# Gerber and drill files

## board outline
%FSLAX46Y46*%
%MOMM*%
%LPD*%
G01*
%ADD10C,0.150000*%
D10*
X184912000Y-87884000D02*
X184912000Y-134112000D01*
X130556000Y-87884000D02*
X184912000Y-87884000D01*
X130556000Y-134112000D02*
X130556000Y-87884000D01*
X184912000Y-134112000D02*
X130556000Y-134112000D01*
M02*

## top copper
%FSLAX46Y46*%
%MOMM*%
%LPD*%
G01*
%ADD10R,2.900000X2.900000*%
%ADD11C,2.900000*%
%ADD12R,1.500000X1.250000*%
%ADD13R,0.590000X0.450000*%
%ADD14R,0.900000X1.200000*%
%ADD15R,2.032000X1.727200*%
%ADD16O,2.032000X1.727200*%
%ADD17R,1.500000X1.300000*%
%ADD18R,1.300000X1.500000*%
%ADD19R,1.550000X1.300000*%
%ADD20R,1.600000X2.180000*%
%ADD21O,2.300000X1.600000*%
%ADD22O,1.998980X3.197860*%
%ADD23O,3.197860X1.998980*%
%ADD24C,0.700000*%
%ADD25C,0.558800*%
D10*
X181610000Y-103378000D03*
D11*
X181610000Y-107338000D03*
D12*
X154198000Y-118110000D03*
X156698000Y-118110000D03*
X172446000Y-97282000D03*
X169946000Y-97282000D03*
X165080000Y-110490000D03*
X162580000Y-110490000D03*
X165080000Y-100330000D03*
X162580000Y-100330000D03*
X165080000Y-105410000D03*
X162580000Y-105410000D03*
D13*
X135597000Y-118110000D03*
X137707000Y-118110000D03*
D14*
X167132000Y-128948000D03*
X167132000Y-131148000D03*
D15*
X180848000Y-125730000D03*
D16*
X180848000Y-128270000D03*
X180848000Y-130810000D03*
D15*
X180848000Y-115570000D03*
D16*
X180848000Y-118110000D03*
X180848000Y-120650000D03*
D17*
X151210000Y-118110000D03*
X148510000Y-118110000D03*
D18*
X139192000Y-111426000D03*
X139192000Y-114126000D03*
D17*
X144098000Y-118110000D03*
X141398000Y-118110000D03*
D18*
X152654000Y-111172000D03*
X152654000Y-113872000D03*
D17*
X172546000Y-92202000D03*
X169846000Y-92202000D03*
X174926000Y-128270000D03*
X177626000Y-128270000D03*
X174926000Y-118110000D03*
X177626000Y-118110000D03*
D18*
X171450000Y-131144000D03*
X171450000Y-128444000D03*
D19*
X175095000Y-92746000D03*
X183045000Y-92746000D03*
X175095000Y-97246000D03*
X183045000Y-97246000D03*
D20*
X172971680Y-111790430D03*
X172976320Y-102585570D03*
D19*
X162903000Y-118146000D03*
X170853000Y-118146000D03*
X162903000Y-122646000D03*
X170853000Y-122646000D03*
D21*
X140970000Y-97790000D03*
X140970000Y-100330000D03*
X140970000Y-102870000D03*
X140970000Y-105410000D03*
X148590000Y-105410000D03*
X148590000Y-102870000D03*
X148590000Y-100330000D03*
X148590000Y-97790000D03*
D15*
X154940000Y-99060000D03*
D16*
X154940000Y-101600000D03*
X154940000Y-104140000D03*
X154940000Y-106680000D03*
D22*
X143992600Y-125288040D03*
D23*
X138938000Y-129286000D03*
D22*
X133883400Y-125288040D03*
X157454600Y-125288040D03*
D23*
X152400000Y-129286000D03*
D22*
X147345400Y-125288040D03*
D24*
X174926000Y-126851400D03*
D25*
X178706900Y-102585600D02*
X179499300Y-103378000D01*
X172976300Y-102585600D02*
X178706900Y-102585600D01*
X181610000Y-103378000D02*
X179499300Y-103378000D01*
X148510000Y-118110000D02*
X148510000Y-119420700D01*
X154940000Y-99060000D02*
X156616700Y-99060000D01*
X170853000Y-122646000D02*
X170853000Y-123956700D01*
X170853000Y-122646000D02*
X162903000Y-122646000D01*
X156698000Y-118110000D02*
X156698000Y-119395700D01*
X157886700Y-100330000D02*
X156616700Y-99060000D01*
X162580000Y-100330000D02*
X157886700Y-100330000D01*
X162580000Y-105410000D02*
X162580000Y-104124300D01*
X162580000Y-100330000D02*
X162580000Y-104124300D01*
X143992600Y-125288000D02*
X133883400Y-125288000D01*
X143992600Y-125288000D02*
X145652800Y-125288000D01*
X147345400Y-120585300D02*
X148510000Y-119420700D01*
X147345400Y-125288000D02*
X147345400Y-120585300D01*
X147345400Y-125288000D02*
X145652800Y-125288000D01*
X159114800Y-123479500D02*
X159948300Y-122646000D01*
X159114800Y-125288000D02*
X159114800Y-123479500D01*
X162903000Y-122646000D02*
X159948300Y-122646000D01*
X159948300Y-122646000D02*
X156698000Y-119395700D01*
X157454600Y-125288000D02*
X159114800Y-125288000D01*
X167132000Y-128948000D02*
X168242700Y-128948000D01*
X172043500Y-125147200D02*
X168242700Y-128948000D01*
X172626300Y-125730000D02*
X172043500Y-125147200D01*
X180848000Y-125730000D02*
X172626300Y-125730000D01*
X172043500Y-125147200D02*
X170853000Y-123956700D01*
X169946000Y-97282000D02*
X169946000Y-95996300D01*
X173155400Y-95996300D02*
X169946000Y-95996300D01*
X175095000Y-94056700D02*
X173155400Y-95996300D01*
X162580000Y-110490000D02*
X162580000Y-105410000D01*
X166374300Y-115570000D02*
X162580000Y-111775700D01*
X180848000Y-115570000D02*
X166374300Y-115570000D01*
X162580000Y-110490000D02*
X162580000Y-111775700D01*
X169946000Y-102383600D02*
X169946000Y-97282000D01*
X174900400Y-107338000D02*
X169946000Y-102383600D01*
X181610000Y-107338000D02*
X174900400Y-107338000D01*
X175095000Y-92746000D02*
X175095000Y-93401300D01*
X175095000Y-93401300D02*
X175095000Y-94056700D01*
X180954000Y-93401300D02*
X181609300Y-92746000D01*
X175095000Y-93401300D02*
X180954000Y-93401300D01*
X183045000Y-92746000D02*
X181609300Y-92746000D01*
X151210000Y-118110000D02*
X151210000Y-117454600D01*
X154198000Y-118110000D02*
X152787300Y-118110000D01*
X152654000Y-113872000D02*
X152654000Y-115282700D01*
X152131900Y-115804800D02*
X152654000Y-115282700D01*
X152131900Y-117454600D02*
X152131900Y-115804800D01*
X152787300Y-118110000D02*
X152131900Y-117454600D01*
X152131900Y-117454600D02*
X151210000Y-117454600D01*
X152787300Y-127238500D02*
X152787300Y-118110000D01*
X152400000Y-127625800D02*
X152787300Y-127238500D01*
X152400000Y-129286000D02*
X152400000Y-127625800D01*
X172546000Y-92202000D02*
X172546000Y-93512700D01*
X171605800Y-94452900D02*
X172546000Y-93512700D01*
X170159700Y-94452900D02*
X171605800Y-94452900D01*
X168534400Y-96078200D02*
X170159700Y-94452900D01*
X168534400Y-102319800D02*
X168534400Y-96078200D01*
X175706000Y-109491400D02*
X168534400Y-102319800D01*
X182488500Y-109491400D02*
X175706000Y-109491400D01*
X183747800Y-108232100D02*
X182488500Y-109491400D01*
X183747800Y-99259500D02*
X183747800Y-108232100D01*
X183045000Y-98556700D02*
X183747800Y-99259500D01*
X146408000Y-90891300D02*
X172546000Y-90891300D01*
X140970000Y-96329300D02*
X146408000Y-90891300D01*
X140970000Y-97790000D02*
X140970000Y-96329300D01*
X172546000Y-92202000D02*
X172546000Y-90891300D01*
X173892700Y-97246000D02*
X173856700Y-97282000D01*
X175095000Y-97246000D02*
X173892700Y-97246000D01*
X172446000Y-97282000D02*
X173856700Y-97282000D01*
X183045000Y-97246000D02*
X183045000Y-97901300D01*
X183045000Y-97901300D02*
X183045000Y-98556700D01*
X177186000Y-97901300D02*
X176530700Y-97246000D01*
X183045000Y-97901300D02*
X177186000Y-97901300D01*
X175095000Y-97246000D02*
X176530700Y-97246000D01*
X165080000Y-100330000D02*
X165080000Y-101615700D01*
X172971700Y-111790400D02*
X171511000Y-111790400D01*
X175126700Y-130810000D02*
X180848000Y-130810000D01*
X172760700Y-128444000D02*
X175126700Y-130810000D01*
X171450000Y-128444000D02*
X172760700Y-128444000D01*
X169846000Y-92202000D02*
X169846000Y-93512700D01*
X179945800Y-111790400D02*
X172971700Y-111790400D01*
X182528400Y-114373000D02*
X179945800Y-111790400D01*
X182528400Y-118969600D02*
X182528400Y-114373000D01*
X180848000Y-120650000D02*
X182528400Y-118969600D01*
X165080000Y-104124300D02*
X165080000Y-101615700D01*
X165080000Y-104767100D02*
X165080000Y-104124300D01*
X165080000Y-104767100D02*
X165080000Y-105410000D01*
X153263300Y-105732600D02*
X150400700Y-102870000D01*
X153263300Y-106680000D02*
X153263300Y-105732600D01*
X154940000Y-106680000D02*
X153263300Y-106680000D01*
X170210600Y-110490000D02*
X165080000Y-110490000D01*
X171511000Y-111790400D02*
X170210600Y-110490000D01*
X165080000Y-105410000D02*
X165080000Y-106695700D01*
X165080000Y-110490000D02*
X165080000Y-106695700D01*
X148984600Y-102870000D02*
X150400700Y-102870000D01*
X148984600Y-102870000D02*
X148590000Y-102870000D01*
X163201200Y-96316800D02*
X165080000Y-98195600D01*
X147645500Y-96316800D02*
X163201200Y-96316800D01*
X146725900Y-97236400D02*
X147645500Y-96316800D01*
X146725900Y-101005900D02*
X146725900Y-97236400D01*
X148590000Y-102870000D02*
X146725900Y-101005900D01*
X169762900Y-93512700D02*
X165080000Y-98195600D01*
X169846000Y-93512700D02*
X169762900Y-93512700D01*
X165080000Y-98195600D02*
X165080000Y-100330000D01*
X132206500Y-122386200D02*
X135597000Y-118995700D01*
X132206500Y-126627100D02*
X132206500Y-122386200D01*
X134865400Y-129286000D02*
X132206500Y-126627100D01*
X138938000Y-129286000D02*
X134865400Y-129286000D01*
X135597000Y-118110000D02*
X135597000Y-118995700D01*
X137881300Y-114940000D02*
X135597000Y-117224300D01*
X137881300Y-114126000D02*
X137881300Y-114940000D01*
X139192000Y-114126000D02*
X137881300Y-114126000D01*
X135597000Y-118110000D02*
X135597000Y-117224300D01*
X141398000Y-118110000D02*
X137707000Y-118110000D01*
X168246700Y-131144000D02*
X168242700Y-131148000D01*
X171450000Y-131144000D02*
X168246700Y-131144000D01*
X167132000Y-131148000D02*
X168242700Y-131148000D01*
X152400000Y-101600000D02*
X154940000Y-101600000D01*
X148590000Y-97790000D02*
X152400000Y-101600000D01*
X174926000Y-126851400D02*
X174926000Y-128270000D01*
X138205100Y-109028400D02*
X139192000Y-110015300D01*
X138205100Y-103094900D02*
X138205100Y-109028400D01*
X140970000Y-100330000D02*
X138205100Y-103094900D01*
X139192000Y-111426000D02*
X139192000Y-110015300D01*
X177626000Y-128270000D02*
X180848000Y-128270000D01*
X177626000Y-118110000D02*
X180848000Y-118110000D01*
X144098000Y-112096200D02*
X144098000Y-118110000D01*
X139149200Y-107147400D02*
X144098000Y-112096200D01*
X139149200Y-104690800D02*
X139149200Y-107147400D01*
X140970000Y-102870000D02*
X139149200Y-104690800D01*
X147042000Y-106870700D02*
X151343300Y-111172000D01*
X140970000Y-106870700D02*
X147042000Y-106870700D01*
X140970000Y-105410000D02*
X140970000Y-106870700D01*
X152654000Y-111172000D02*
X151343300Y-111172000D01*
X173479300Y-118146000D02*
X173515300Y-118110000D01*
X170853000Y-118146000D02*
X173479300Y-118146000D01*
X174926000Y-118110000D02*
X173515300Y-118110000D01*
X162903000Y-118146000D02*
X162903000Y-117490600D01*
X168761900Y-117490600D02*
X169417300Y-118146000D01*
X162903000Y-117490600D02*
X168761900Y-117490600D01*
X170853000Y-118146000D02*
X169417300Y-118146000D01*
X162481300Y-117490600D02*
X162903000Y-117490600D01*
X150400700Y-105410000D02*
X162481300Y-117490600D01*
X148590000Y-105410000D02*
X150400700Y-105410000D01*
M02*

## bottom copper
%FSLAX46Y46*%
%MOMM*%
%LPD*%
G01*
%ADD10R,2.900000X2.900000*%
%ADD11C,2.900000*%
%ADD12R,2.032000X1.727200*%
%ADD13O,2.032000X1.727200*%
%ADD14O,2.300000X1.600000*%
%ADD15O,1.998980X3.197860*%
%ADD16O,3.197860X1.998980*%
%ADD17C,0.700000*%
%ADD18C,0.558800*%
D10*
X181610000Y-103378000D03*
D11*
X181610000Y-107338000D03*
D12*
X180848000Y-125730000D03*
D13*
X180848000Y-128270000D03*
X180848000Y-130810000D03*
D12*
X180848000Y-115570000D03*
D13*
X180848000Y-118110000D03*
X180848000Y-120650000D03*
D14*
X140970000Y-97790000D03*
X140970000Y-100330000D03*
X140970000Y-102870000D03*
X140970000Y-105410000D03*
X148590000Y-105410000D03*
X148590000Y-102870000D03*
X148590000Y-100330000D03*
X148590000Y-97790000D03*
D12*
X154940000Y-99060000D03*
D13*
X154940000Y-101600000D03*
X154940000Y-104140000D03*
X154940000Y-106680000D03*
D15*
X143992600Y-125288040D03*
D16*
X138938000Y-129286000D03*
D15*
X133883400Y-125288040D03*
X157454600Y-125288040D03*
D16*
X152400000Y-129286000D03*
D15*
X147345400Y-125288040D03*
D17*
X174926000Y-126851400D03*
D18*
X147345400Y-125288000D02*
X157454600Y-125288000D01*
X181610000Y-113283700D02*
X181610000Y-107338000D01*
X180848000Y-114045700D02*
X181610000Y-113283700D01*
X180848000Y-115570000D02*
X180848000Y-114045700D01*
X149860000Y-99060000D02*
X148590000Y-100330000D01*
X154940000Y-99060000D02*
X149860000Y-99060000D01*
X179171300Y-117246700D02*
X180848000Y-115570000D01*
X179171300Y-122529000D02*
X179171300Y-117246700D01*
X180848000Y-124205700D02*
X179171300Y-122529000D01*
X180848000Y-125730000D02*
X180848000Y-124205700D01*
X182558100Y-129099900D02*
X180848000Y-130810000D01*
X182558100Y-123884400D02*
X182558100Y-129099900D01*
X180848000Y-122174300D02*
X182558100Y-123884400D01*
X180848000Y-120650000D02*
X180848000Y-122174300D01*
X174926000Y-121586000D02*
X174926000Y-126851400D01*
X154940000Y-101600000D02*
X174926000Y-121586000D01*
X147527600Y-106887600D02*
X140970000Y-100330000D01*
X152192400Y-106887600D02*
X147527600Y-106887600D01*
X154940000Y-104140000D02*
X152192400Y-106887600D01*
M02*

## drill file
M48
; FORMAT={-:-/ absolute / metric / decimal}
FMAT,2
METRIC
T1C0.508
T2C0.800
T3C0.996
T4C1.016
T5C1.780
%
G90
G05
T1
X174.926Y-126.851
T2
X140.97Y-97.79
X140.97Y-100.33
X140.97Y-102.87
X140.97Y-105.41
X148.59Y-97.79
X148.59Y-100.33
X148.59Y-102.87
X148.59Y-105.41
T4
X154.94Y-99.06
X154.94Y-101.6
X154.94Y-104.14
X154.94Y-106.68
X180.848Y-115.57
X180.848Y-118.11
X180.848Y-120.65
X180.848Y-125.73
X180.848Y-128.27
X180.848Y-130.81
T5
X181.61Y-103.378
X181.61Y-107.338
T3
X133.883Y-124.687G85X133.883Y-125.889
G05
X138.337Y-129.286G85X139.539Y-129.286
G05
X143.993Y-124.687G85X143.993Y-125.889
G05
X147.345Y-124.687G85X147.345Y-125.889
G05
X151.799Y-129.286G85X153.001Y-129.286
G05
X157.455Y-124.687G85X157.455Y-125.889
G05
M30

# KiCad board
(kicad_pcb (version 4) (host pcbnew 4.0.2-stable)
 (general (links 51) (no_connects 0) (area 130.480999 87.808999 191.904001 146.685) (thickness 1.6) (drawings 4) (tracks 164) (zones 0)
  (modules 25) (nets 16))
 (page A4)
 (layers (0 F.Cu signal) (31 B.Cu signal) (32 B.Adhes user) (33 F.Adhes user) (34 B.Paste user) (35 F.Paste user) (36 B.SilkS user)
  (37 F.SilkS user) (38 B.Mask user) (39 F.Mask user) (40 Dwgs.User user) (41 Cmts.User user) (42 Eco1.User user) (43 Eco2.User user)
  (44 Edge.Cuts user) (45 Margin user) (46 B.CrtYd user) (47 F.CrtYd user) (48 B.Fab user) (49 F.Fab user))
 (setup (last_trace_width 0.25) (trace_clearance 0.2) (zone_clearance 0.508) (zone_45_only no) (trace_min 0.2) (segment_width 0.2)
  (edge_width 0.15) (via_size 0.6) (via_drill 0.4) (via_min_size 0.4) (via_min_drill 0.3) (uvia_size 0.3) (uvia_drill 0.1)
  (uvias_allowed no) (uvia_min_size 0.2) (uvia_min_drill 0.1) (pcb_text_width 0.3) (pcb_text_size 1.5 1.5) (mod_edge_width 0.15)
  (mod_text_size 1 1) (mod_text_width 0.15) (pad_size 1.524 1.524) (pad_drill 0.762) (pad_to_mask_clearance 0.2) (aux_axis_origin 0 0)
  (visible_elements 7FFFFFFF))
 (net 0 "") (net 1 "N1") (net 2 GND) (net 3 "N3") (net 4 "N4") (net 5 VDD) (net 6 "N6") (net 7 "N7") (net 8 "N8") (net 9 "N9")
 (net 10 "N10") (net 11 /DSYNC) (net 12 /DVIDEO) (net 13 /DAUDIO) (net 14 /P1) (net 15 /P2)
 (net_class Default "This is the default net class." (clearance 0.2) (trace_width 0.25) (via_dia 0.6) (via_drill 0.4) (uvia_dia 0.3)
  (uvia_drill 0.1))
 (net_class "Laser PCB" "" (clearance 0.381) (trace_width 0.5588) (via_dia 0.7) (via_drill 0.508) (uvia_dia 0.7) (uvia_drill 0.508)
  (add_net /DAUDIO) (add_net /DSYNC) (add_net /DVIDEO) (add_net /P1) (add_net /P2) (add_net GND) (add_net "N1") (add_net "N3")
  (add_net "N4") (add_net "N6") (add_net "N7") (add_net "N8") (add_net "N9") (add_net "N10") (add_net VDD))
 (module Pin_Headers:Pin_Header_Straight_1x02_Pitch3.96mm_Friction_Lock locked (layer F.Cu) (at 181.61 103.378 270)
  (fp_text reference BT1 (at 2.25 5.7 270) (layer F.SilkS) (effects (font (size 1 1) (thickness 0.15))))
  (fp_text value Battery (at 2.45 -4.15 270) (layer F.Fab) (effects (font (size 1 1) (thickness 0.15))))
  (pad 1 thru_hole rect (at 0 0 270) (size 2.9 2.9) (drill 1.78) (layers *.Cu *.Mask F.SilkS) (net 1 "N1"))
  (pad 2 thru_hole circle (at 3.96 0 270) (size 2.9 2.9) (drill 1.78) (layers *.Cu *.Mask F.SilkS) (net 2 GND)))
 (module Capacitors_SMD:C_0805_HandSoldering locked (layer F.Cu) (at 155.448 118.11)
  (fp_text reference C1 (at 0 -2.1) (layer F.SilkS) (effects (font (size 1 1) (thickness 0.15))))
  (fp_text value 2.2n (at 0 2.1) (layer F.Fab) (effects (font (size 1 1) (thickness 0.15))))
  (pad 1 smd rect (at -1.25 0) (size 1.5 1.25) (layers F.Cu F.Paste F.Mask) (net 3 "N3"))
  (pad 2 smd rect (at 1.25 0) (size 1.5 1.25) (layers F.Cu F.Paste F.Mask) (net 2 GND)))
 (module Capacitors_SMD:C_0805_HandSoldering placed (layer F.Cu) (at 171.196 97.282 180)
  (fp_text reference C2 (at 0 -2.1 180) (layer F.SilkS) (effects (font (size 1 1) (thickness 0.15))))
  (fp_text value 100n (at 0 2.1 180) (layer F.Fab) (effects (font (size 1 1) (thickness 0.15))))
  (pad 1 smd rect (at -1.25 0 180) (size 1.5 1.25) (layers F.Cu F.Paste F.Mask) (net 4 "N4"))
  (pad 2 smd rect (at 1.25 0 180) (size 1.5 1.25) (layers F.Cu F.Paste F.Mask) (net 2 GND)))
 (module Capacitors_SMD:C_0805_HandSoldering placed (layer F.Cu) (at 163.83 110.49 180)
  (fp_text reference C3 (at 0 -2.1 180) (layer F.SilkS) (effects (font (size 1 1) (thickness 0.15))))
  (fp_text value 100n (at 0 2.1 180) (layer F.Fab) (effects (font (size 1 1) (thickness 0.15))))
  (pad 1 smd rect (at -1.25 0 180) (size 1.5 1.25) (layers F.Cu F.Paste F.Mask) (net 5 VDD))
  (pad 2 smd rect (at 1.25 0 180) (size 1.5 1.25) (layers F.Cu F.Paste F.Mask) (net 2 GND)))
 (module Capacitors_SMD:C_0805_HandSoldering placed (layer F.Cu) (at 163.83 100.33 180)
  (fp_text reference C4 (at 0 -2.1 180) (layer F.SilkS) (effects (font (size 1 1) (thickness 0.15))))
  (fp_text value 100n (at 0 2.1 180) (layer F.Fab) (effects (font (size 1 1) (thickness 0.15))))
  (pad 1 smd rect (at -1.25 0 180) (size 1.5 1.25) (layers F.Cu F.Paste F.Mask) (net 5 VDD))
  (pad 2 smd rect (at 1.25 0 180) (size 1.5 1.25) (layers F.Cu F.Paste F.Mask) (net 2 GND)))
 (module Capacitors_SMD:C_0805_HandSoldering (layer F.Cu) (at 163.83 105.41 180)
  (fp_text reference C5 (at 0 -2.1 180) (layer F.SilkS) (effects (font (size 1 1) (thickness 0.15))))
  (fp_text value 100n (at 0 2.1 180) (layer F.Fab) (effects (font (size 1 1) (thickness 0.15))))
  (pad 1 smd rect (at -1.25 0 180) (size 1.5 1.25) (layers F.Cu F.Paste F.Mask) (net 5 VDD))
  (pad 2 smd rect (at 1.25 0 180) (size 1.5 1.25) (layers F.Cu F.Paste F.Mask) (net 2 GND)))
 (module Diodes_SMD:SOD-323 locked (layer F.Cu) (at 136.652 118.11)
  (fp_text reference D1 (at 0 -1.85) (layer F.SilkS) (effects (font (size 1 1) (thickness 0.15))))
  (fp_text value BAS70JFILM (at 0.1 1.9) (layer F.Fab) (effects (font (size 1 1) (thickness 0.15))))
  (pad 1 smd rect (at -1.055 0) (size 0.59 0.45) (layers F.Cu F.Paste F.Mask) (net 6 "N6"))
  (pad 2 smd rect (at 1.055 0) (size 0.59 0.45) (layers F.Cu F.Paste F.Mask) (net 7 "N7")))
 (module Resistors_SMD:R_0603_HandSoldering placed (layer F.Cu) (at 167.132 130.048 270)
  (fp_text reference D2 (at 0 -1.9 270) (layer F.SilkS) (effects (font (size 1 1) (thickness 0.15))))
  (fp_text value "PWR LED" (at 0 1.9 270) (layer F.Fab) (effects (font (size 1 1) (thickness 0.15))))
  (pad 1 smd rect (at -1.1 0 270) (size 1.2 0.9) (layers F.Cu F.Paste F.Mask) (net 2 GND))
  (pad 2 smd rect (at 1.1 0 270) (size 1.2 0.9) (layers F.Cu F.Paste F.Mask) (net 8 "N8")))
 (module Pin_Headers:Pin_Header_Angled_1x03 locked (layer F.Cu) (at 180.848 125.73)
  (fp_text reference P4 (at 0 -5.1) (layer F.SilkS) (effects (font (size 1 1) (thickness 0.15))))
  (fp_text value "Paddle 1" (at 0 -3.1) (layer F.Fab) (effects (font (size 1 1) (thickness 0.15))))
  (pad 1 thru_hole rect (at 0 0) (size 2.032 1.7272) (drill 1.016) (layers *.Cu *.Mask F.SilkS) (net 2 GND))
  (pad 2 thru_hole oval (at 0 2.54) (size 2.032 1.7272) (drill 1.016) (layers *.Cu *.Mask F.SilkS) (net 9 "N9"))
  (pad 3 thru_hole oval (at 0 5.08) (size 2.032 1.7272) (drill 1.016) (layers *.Cu *.Mask F.SilkS) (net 5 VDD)))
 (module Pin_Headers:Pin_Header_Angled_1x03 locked (layer F.Cu) (at 180.848 115.57)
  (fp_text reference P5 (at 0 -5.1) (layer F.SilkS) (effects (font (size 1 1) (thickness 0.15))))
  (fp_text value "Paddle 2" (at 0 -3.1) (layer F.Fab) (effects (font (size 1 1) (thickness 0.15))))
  (pad 1 thru_hole rect (at 0 0) (size 2.032 1.7272) (drill 1.016) (layers *.Cu *.Mask F.SilkS) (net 2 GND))
  (pad 2 thru_hole oval (at 0 2.54) (size 2.032 1.7272) (drill 1.016) (layers *.Cu *.Mask F.SilkS) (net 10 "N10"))
  (pad 3 thru_hole oval (at 0 5.08) (size 2.032 1.7272) (drill 1.016) (layers *.Cu *.Mask F.SilkS) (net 5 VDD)))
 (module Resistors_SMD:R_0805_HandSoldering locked (layer F.Cu) (at 149.86 118.11 180)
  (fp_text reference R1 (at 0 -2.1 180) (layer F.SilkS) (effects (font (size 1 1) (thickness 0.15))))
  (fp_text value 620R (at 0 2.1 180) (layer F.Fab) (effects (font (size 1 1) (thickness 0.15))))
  (pad 1 smd rect (at -1.35 0 180) (size 1.5 1.3) (layers F.Cu F.Paste F.Mask) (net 3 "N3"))
  (pad 2 smd rect (at 1.35 0 180) (size 1.5 1.3) (layers F.Cu F.Paste F.Mask) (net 2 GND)))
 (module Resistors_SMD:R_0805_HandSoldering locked (layer F.Cu) (at 139.192 112.776 270)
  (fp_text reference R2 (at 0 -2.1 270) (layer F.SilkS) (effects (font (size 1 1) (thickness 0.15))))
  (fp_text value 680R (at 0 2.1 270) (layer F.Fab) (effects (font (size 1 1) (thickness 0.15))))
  (pad 1 smd rect (at -1.35 0 270) (size 1.5 1.3) (layers F.Cu F.Paste F.Mask) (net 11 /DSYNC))
  (pad 2 smd rect (at 1.35 0 270) (size 1.5 1.3) (layers F.Cu F.Paste F.Mask) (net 6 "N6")))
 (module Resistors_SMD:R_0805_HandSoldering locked (layer F.Cu) (at 142.748 118.11 180)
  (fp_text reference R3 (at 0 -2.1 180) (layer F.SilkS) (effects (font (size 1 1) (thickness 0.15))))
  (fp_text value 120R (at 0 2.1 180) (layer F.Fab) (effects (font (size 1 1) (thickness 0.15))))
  (pad 1 smd rect (at -1.35 0 180) (size 1.5 1.3) (layers F.Cu F.Paste F.Mask) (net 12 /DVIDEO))
  (pad 2 smd rect (at 1.35 0 180) (size 1.5 1.3) (layers F.Cu F.Paste F.Mask) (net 7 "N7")))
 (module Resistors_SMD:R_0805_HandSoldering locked (layer F.Cu) (at 152.654 112.522 270)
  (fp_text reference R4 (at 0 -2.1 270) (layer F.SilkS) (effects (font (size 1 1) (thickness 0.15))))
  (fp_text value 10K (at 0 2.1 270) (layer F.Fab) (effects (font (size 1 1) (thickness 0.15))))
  (pad 1 smd rect (at -1.35 0 270) (size 1.5 1.3) (layers F.Cu F.Paste F.Mask) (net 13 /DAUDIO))
  (pad 2 smd rect (at 1.35 0 270) (size 1.5 1.3) (layers F.Cu F.Paste F.Mask) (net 3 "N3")))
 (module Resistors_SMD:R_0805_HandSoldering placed (layer F.Cu) (at 171.196 92.202 180)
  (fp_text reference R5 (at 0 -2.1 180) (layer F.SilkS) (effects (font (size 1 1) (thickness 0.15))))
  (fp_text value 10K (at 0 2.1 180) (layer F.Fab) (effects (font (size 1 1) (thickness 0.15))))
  (pad 1 smd rect (at -1.35 0 180) (size 1.5 1.3) (layers F.Cu F.Paste F.Mask) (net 4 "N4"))
  (pad 2 smd rect (at 1.35 0 180) (size 1.5 1.3) (layers F.Cu F.Paste F.Mask) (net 5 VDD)))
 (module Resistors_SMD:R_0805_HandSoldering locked (layer F.Cu) (at 176.276 128.27)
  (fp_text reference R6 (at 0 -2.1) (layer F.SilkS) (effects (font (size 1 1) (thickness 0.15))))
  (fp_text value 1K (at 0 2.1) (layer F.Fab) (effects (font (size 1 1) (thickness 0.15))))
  (pad 1 smd rect (at -1.35 0) (size 1.5 1.3) (layers F.Cu F.Paste F.Mask) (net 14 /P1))
  (pad 2 smd rect (at 1.35 0) (size 1.5 1.3) (layers F.Cu F.Paste F.Mask) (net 9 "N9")))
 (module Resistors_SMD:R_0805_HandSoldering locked (layer F.Cu) (at 176.276 118.11)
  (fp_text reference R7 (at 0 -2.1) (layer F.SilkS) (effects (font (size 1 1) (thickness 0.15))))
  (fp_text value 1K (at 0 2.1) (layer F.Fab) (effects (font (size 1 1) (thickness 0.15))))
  (pad 1 smd rect (at -1.35 0) (size 1.5 1.3) (layers F.Cu F.Paste F.Mask) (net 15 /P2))
  (pad 2 smd rect (at 1.35 0) (size 1.5 1.3) (layers F.Cu F.Paste F.Mask) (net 10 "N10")))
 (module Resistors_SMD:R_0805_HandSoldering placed (layer F.Cu) (at 171.45 129.794 90)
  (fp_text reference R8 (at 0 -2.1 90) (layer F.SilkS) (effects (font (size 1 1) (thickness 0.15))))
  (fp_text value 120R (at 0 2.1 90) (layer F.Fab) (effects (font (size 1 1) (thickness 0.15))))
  (pad 1 smd rect (at -1.35 0 90) (size 1.5 1.3) (layers F.Cu F.Paste F.Mask) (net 8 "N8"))
  (pad 2 smd rect (at 1.35 0 90) (size 1.5 1.3) (layers F.Cu F.Paste F.Mask) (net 5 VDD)))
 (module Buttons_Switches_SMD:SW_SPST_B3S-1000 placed (layer F.Cu) (at 179.07 94.996)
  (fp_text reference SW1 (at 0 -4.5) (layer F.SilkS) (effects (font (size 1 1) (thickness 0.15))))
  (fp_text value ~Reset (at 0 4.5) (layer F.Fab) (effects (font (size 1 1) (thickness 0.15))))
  (pad 1 smd rect (at -3.975 -2.25) (size 1.55 1.3) (layers F.Cu F.Paste F.Mask) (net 2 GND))
  (pad 1 smd rect (at 3.975 -2.25) (size 1.55 1.3) (layers F.Cu F.Paste F.Mask) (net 2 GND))
  (pad 2 smd rect (at -3.975 2.25) (size 1.55 1.3) (layers F.Cu F.Paste F.Mask) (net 4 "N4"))
  (pad 2 smd rect (at 3.975 2.25) (size 1.55 1.3) (layers F.Cu F.Paste F.Mask) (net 4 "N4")))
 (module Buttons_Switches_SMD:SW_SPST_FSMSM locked (layer F.Cu) (at 172.974 107.188 90)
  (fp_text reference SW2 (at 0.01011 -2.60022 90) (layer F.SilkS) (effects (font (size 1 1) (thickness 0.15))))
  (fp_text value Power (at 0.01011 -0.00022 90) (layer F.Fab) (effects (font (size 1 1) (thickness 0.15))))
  (pad 1 smd rect (at -4.60243 -0.00232 90) (size 2.18 1.6) (layers F.Cu F.Paste F.Mask) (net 5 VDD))
  (pad 2 smd rect (at 4.60243 0.00232 90) (size 2.18 1.6) (layers F.Cu F.Paste F.Mask) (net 1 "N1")))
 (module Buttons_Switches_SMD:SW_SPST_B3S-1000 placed (layer F.Cu) (at 166.878 120.396)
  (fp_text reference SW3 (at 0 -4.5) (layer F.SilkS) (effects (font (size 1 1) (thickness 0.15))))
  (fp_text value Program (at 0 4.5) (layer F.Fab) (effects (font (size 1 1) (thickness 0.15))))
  (pad 1 smd rect (at -3.975 -2.25) (size 1.55 1.3) (layers F.Cu F.Paste F.Mask) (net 15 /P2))
  (pad 1 smd rect (at 3.975 -2.25) (size 1.55 1.3) (layers F.Cu F.Paste F.Mask) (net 15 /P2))
  (pad 2 smd rect (at -3.975 2.25) (size 1.55 1.3) (layers F.Cu F.Paste F.Mask) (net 2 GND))
  (pad 2 smd rect (at 3.975 2.25) (size 1.55 1.3) (layers F.Cu F.Paste F.Mask) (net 2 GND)))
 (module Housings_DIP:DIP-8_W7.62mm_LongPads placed (layer F.Cu) (at 140.97 97.79)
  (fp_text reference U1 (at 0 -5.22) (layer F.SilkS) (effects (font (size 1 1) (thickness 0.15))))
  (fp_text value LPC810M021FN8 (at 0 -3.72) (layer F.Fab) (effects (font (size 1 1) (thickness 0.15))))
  (pad 1 thru_hole oval (at 0 0) (size 2.3 1.6) (drill 0.8) (layers *.Cu *.Mask F.SilkS) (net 4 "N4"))
  (pad 2 thru_hole oval (at 0 2.54) (size 2.3 1.6) (drill 0.8) (layers *.Cu *.Mask F.SilkS) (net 11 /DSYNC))
  (pad 3 thru_hole oval (at 0 5.08) (size 2.3 1.6) (drill 0.8) (layers *.Cu *.Mask F.SilkS) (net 12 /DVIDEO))
  (pad 4 thru_hole oval (at 0 7.62) (size 2.3 1.6) (drill 0.8) (layers *.Cu *.Mask F.SilkS) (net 13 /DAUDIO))
  (pad 5 thru_hole oval (at 7.62 7.62) (size 2.3 1.6) (drill 0.8) (layers *.Cu *.Mask F.SilkS) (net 15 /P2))
  (pad 6 thru_hole oval (at 7.62 5.08) (size 2.3 1.6) (drill 0.8) (layers *.Cu *.Mask F.SilkS) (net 5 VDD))
  (pad 7 thru_hole oval (at 7.62 2.54) (size 2.3 1.6) (drill 0.8) (layers *.Cu *.Mask F.SilkS) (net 2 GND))
  (pad 8 thru_hole oval (at 7.62 0) (size 2.3 1.6) (drill 0.8) (layers *.Cu *.Mask F.SilkS) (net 14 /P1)))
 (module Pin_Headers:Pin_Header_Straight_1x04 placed (layer F.Cu) (at 154.94 99.06)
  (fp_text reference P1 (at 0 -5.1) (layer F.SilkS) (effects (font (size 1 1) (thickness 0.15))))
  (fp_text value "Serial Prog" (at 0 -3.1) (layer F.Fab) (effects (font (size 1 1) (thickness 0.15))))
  (pad 1 thru_hole rect (at 0 0) (size 2.032 1.7272) (drill 1.016) (layers *.Cu *.Mask F.SilkS) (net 2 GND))
  (pad 2 thru_hole oval (at 0 2.54) (size 2.032 1.7272) (drill 1.016) (layers *.Cu *.Mask F.SilkS) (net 14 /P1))
  (pad 3 thru_hole oval (at 0 5.08) (size 2.032 1.7272) (drill 1.016) (layers *.Cu *.Mask F.SilkS) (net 11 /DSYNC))
  (pad 4 thru_hole oval (at 0 7.62) (size 2.032 1.7272) (drill 1.016) (layers *.Cu *.Mask F.SilkS) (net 5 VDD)))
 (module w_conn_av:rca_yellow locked (layer F.Cu) (at 138.938 129.286)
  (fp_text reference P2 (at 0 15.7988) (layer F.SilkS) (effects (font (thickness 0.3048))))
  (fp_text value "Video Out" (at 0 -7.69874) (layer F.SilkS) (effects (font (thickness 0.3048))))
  (pad 2 thru_hole oval (at 5.0546 -3.99796) (size 1.99898 3.19786) (drill oval 0.99568 2.1971) (layers *.Cu *.Mask F.SilkS) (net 2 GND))
  (pad 1 thru_hole oval (at 0 0) (size 3.19786 1.99898) (drill oval 2.1971 0.99568) (layers *.Cu *.Mask F.SilkS) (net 6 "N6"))
  (pad 2 thru_hole oval (at -5.0546 -3.99796) (size 1.99898 3.19786) (drill oval 0.99568 2.1971) (layers *.Cu *.Mask F.SilkS) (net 2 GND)))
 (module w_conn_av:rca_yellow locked (layer F.Cu) (at 152.4 129.286)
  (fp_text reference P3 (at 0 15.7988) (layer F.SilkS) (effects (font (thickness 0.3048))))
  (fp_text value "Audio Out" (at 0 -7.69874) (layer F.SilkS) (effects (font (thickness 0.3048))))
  (pad 2 thru_hole oval (at 5.0546 -3.99796) (size 1.99898 3.19786) (drill oval 0.99568 2.1971) (layers *.Cu *.Mask F.SilkS) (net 2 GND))
  (pad 1 thru_hole oval (at 0 0) (size 3.19786 1.99898) (drill oval 2.1971 0.99568) (layers *.Cu *.Mask F.SilkS) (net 3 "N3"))
  (pad 2 thru_hole oval (at -5.0546 -3.99796) (size 1.99898 3.19786) (drill oval 0.99568 2.1971) (layers *.Cu *.Mask F.SilkS) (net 2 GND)))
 (gr_line (start 184.912 87.884) (end 184.912 134.112) (angle 90) (layer Edge.Cuts) (width 0.15))
 (gr_line (start 130.556 87.884) (end 184.912 87.884) (angle 90) (layer Edge.Cuts) (width 0.15))
 (gr_line (start 130.556 134.112) (end 130.556 87.884) (angle 90) (layer Edge.Cuts) (width 0.15))
 (gr_line (start 184.912 134.112) (end 130.556 134.112) (angle 90) (layer Edge.Cuts) (width 0.15))
 (segment (start 178.7069 102.5856) (end 179.4993 103.378) (width 0.5588) (layer F.Cu) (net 1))
 (segment (start 172.9763 102.5856) (end 178.7069 102.5856) (width 0.5588) (layer F.Cu) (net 1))
 (segment (start 181.61 103.378) (end 179.4993 103.378) (width 0.5588) (layer F.Cu) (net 1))
 (segment (start 148.51 118.11) (end 148.51 119.4207) (width 0.5588) (layer F.Cu) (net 2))
 (segment (start 154.94 99.06) (end 156.6167 99.06) (width 0.5588) (layer F.Cu) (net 2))
 (segment (start 170.853 122.646) (end 170.853 123.9567) (width 0.5588) (layer F.Cu) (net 2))
 (segment (start 170.853 122.646) (end 162.903 122.646) (width 0.5588) (layer F.Cu) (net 2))
 (segment (start 156.698 118.11) (end 156.698 119.3957) (width 0.5588) (layer F.Cu) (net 2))
 (segment (start 157.8867 100.33) (end 156.6167 99.06) (width 0.5588) (layer F.Cu) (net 2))
 (segment (start 162.58 100.33) (end 157.8867 100.33) (width 0.5588) (layer F.Cu) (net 2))
 (segment (start 162.58 105.41) (end 162.58 104.1243) (width 0.5588) (layer F.Cu) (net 2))
 (segment (start 162.58 100.33) (end 162.58 104.1243) (width 0.5588) (layer F.Cu) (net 2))
 (segment (start 143.9926 125.288) (end 133.8834 125.288) (width 0.5588) (layer F.Cu) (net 2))
 (segment (start 143.9926 125.288) (end 145.6528 125.288) (width 0.5588) (layer F.Cu) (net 2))
 (segment (start 147.3454 120.5853) (end 148.51 119.4207) (width 0.5588) (layer F.Cu) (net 2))
 (segment (start 147.3454 125.288) (end 147.3454 120.5853) (width 0.5588) (layer F.Cu) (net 2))
 (segment (start 147.3454 125.288) (end 145.6528 125.288) (width 0.5588) (layer F.Cu) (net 2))
 (segment (start 147.3454 125.288) (end 157.4546 125.288) (width 0.5588) (layer B.Cu) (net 2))
 (segment (start 159.1148 123.4795) (end 159.9483 122.646) (width 0.5588) (layer F.Cu) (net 2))
 (segment (start 159.1148 125.288) (end 159.1148 123.4795) (width 0.5588) (layer F.Cu) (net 2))
 (segment (start 162.903 122.646) (end 159.9483 122.646) (width 0.5588) (layer F.Cu) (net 2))
 (segment (start 159.9483 122.646) (end 156.698 119.3957) (width 0.5588) (layer F.Cu) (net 2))
 (segment (start 157.4546 125.288) (end 159.1148 125.288) (width 0.5588) (layer F.Cu) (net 2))
 (segment (start 167.132 128.948) (end 168.2427 128.948) (width 0.5588) (layer F.Cu) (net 2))
 (segment (start 172.0435 125.1472) (end 168.2427 128.948) (width 0.5588) (layer F.Cu) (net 2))
 (segment (start 172.6263 125.73) (end 172.0435 125.1472) (width 0.5588) (layer F.Cu) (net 2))
 (segment (start 180.848 125.73) (end 172.6263 125.73) (width 0.5588) (layer F.Cu) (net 2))
 (segment (start 172.0435 125.1472) (end 170.853 123.9567) (width 0.5588) (layer F.Cu) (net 2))
 (segment (start 169.946 97.282) (end 169.946 95.9963) (width 0.5588) (layer F.Cu) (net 2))
 (segment (start 173.1554 95.9963) (end 169.946 95.9963) (width 0.5588) (layer F.Cu) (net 2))
 (segment (start 175.095 94.0567) (end 173.1554 95.9963) (width 0.5588) (layer F.Cu) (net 2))
 (segment (start 181.61 113.2837) (end 181.61 107.338) (width 0.5588) (layer B.Cu) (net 2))
 (segment (start 180.848 114.0457) (end 181.61 113.2837) (width 0.5588) (layer B.Cu) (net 2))
 (segment (start 180.848 115.57) (end 180.848 114.0457) (width 0.5588) (layer B.Cu) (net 2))
 (segment (start 162.58 110.49) (end 162.58 105.41) (width 0.5588) (layer F.Cu) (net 2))
 (segment (start 149.86 99.06) (end 148.59 100.33) (width 0.5588) (layer B.Cu) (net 2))
 (segment (start 154.94 99.06) (end 149.86 99.06) (width 0.5588) (layer B.Cu) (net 2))
 (segment (start 166.3743 115.57) (end 162.58 111.7757) (width 0.5588) (layer F.Cu) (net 2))
 (segment (start 180.848 115.57) (end 166.3743 115.57) (width 0.5588) (layer F.Cu) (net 2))
 (segment (start 162.58 110.49) (end 162.58 111.7757) (width 0.5588) (layer F.Cu) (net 2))
 (segment (start 179.1713 117.2467) (end 180.848 115.57) (width 0.5588) (layer B.Cu) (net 2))
 (segment (start 179.1713 122.529) (end 179.1713 117.2467) (width 0.5588) (layer B.Cu) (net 2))
 (segment (start 180.848 124.2057) (end 179.1713 122.529) (width 0.5588) (layer B.Cu) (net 2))
 (segment (start 180.848 125.73) (end 180.848 124.2057) (width 0.5588) (layer B.Cu) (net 2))
 (segment (start 169.946 102.3836) (end 169.946 97.282) (width 0.5588) (layer F.Cu) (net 2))
 (segment (start 174.9004 107.338) (end 169.946 102.3836) (width 0.5588) (layer F.Cu) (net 2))
 (segment (start 181.61 107.338) (end 174.9004 107.338) (width 0.5588) (layer F.Cu) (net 2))
 (segment (start 175.095 92.746) (end 175.095 93.4013) (width 0.5588) (layer F.Cu) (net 2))
 (segment (start 175.095 93.4013) (end 175.095 94.0567) (width 0.5588) (layer F.Cu) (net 2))
 (segment (start 180.954 93.4013) (end 181.6093 92.746) (width 0.5588) (layer F.Cu) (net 2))
 (segment (start 175.095 93.4013) (end 180.954 93.4013) (width 0.5588) (layer F.Cu) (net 2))
 (segment (start 183.045 92.746) (end 181.6093 92.746) (width 0.5588) (layer F.Cu) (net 2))
 (segment (start 151.21 118.11) (end 151.21 117.4546) (width 0.5588) (layer F.Cu) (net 3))
 (segment (start 154.198 118.11) (end 152.7873 118.11) (width 0.5588) (layer F.Cu) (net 3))
 (segment (start 152.654 113.872) (end 152.654 115.2827) (width 0.5588) (layer F.Cu) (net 3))
 (segment (start 152.1319 115.8048) (end 152.654 115.2827) (width 0.5588) (layer F.Cu) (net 3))
 (segment (start 152.1319 117.4546) (end 152.1319 115.8048) (width 0.5588) (layer F.Cu) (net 3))
 (segment (start 152.7873 118.11) (end 152.1319 117.4546) (width 0.5588) (layer F.Cu) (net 3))
 (segment (start 152.1319 117.4546) (end 151.21 117.4546) (width 0.5588) (layer F.Cu) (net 3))
 (segment (start 152.7873 127.2385) (end 152.7873 118.11) (width 0.5588) (layer F.Cu) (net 3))
 (segment (start 152.4 127.6258) (end 152.7873 127.2385) (width 0.5588) (layer F.Cu) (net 3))
 (segment (start 152.4 129.286) (end 152.4 127.6258) (width 0.5588) (layer F.Cu) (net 3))
 (segment (start 172.546 92.202) (end 172.546 93.5127) (width 0.5588) (layer F.Cu) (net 4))
 (segment (start 171.6058 94.4529) (end 172.546 93.5127) (width 0.5588) (layer F.Cu) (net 4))
 (segment (start 170.1597 94.4529) (end 171.6058 94.4529) (width 0.5588) (layer F.Cu) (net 4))
 (segment (start 168.5344 96.0782) (end 170.1597 94.4529) (width 0.5588) (layer F.Cu) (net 4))
 (segment (start 168.5344 102.3198) (end 168.5344 96.0782) (width 0.5588) (layer F.Cu) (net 4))
 (segment (start 175.706 109.4914) (end 168.5344 102.3198) (width 0.5588) (layer F.Cu) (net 4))
 (segment (start 182.4885 109.4914) (end 175.706 109.4914) (width 0.5588) (layer F.Cu) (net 4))
 (segment (start 183.7478 108.2321) (end 182.4885 109.4914) (width 0.5588) (layer F.Cu) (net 4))
 (segment (start 183.7478 99.2595) (end 183.7478 108.2321) (width 0.5588) (layer F.Cu) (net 4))
 (segment (start 183.045 98.5567) (end 183.7478 99.2595) (width 0.5588) (layer F.Cu) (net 4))
 (segment (start 146.408 90.8913) (end 172.546 90.8913) (width 0.5588) (layer F.Cu) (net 4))
 (segment (start 140.97 96.3293) (end 146.408 90.8913) (width 0.5588) (layer F.Cu) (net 4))
 (segment (start 140.97 97.79) (end 140.97 96.3293) (width 0.5588) (layer F.Cu) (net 4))
 (segment (start 172.546 92.202) (end 172.546 90.8913) (width 0.5588) (layer F.Cu) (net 4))
 (segment (start 173.8927 97.246) (end 173.8567 97.282) (width 0.5588) (layer F.Cu) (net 4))
 (segment (start 175.095 97.246) (end 173.8927 97.246) (width 0.5588) (layer F.Cu) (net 4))
 (segment (start 172.446 97.282) (end 173.8567 97.282) (width 0.5588) (layer F.Cu) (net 4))
 (segment (start 183.045 97.246) (end 183.045 97.9013) (width 0.5588) (layer F.Cu) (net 4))
 (segment (start 183.045 97.9013) (end 183.045 98.5567) (width 0.5588) (layer F.Cu) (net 4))
 (segment (start 177.186 97.9013) (end 176.5307 97.246) (width 0.5588) (layer F.Cu) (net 4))
 (segment (start 183.045 97.9013) (end 177.186 97.9013) (width 0.5588) (layer F.Cu) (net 4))
 (segment (start 175.095 97.246) (end 176.5307 97.246) (width 0.5588) (layer F.Cu) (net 4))
 (segment (start 165.08 100.33) (end 165.08 101.6157) (width 0.5588) (layer F.Cu) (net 5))
 (segment (start 172.9717 111.7904) (end 171.511 111.7904) (width 0.5588) (layer F.Cu) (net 5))
 (segment (start 175.1267 130.81) (end 180.848 130.81) (width 0.5588) (layer F.Cu) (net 5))
 (segment (start 172.7607 128.444) (end 175.1267 130.81) (width 0.5588) (layer F.Cu) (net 5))
 (segment (start 171.45 128.444) (end 172.7607 128.444) (width 0.5588) (layer F.Cu) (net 5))
 (segment (start 169.846 92.202) (end 169.846 93.5127) (width 0.5588) (layer F.Cu) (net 5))
 (segment (start 182.5581 129.0999) (end 180.848 130.81) (width 0.5588) (layer B.Cu) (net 5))
 (segment (start 182.5581 123.8844) (end 182.5581 129.0999) (width 0.5588) (layer B.Cu) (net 5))
 (segment (start 180.848 122.1743) (end 182.5581 123.8844) (width 0.5588) (layer B.Cu) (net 5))
 (segment (start 180.848 120.65) (end 180.848 122.1743) (width 0.5588) (layer B.Cu) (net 5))
 (segment (start 179.9458 111.7904) (end 172.9717 111.7904) (width 0.5588) (layer F.Cu) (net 5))
 (segment (start 182.5284 114.373) (end 179.9458 111.7904) (width 0.5588) (layer F.Cu) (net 5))
 (segment (start 182.5284 118.9696) (end 182.5284 114.373) (width 0.5588) (layer F.Cu) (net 5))
 (segment (start 180.848 120.65) (end 182.5284 118.9696) (width 0.5588) (layer F.Cu) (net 5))
 (segment (start 165.08 104.1243) (end 165.08 101.6157) (width 0.5588) (layer F.Cu) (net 5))
 (segment (start 165.08 104.7671) (end 165.08 104.1243) (width 0.5588) (layer F.Cu) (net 5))
 (segment (start 165.08 104.7671) (end 165.08 105.41) (width 0.5588) (layer F.Cu) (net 5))
 (segment (start 153.2633 105.7326) (end 150.4007 102.87) (width 0.5588) (layer F.Cu) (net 5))
 (segment (start 153.2633 106.68) (end 153.2633 105.7326) (width 0.5588) (layer F.Cu) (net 5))
 (segment (start 154.94 106.68) (end 153.2633 106.68) (width 0.5588) (layer F.Cu) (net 5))
 (segment (start 170.2106 110.49) (end 165.08 110.49) (width 0.5588) (layer F.Cu) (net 5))
 (segment (start 171.511 111.7904) (end 170.2106 110.49) (width 0.5588) (layer F.Cu) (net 5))
 (segment (start 165.08 105.41) (end 165.08 106.6957) (width 0.5588) (layer F.Cu) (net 5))
 (segment (start 165.08 110.49) (end 165.08 106.6957) (width 0.5588) (layer F.Cu) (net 5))
 (segment (start 148.9846 102.87) (end 150.4007 102.87) (width 0.5588) (layer F.Cu) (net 5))
 (segment (start 148.9846 102.87) (end 148.59 102.87) (width 0.5588) (layer F.Cu) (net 5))
 (segment (start 163.2012 96.3168) (end 165.08 98.1956) (width 0.5588) (layer F.Cu) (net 5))
 (segment (start 147.6455 96.3168) (end 163.2012 96.3168) (width 0.5588) (layer F.Cu) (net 5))
 (segment (start 146.7259 97.2364) (end 147.6455 96.3168) (width 0.5588) (layer F.Cu) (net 5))
 (segment (start 146.7259 101.0059) (end 146.7259 97.2364) (width 0.5588) (layer F.Cu) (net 5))
 (segment (start 148.59 102.87) (end 146.7259 101.0059) (width 0.5588) (layer F.Cu) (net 5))
 (segment (start 169.7629 93.5127) (end 165.08 98.1956) (width 0.5588) (layer F.Cu) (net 5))
 (segment (start 169.846 93.5127) (end 169.7629 93.5127) (width 0.5588) (layer F.Cu) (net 5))
 (segment (start 165.08 98.1956) (end 165.08 100.33) (width 0.5588) (layer F.Cu) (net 5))
 (segment (start 132.2065 122.3862) (end 135.597 118.9957) (width 0.5588) (layer F.Cu) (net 6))
 (segment (start 132.2065 126.6271) (end 132.2065 122.3862) (width 0.5588) (layer F.Cu) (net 6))
 (segment (start 134.8654 129.286) (end 132.2065 126.6271) (width 0.5588) (layer F.Cu) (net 6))
 (segment (start 138.938 129.286) (end 134.8654 129.286) (width 0.5588) (layer F.Cu) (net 6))
 (segment (start 135.597 118.11) (end 135.597 118.9957) (width 0.5588) (layer F.Cu) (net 6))
 (segment (start 137.8813 114.94) (end 135.597 117.2243) (width 0.5588) (layer F.Cu) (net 6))
 (segment (start 137.8813 114.126) (end 137.8813 114.94) (width 0.5588) (layer F.Cu) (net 6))
 (segment (start 139.192 114.126) (end 137.8813 114.126) (width 0.5588) (layer F.Cu) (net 6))
 (segment (start 135.597 118.11) (end 135.597 117.2243) (width 0.5588) (layer F.Cu) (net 6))
 (segment (start 141.398 118.11) (end 137.707 118.11) (width 0.5588) (layer F.Cu) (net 7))
 (segment (start 168.2467 131.144) (end 168.2427 131.148) (width 0.5588) (layer F.Cu) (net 8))
 (segment (start 171.45 131.144) (end 168.2467 131.144) (width 0.5588) (layer F.Cu) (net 8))
 (segment (start 167.132 131.148) (end 168.2427 131.148) (width 0.5588) (layer F.Cu) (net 8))
 (via (at 174.926 126.8514) (size 0.7) (drill 0.508) (layers F.Cu B.Cu) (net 14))
 (segment (start 152.4 101.6) (end 154.94 101.6) (width 0.5588) (layer F.Cu) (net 14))
 (segment (start 148.59 97.79) (end 152.4 101.6) (width 0.5588) (layer F.Cu) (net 14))
 (segment (start 174.926 121.586) (end 174.926 126.8514) (width 0.5588) (layer B.Cu) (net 14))
 (segment (start 154.94 101.6) (end 174.926 121.586) (width 0.5588) (layer B.Cu) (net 14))
 (segment (start 174.926 126.8514) (end 174.926 128.27) (width 0.5588) (layer F.Cu) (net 14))
 (segment (start 147.5276 106.8876) (end 140.97 100.33) (width 0.5588) (layer B.Cu) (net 11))
 (segment (start 152.1924 106.8876) (end 147.5276 106.8876) (width 0.5588) (layer B.Cu) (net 11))
 (segment (start 154.94 104.14) (end 152.1924 106.8876) (width 0.5588) (layer B.Cu) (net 11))
 (segment (start 138.2051 109.0284) (end 139.192 110.0153) (width 0.5588) (layer F.Cu) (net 11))
 (segment (start 138.2051 103.0949) (end 138.2051 109.0284) (width 0.5588) (layer F.Cu) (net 11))
 (segment (start 140.97 100.33) (end 138.2051 103.0949) (width 0.5588) (layer F.Cu) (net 11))
 (segment (start 139.192 111.426) (end 139.192 110.0153) (width 0.5588) (layer F.Cu) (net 11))
 (segment (start 177.626 128.27) (end 180.848 128.27) (width 0.5588) (layer F.Cu) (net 9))
 (segment (start 177.626 118.11) (end 180.848 118.11) (width 0.5588) (layer F.Cu) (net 10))
 (segment (start 144.098 112.0962) (end 144.098 118.11) (width 0.5588) (layer F.Cu) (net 12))
 (segment (start 139.1492 107.1474) (end 144.098 112.0962) (width 0.5588) (layer F.Cu) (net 12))
 (segment (start 139.1492 104.6908) (end 139.1492 107.1474) (width 0.5588) (layer F.Cu) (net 12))
 (segment (start 140.97 102.87) (end 139.1492 104.6908) (width 0.5588) (layer F.Cu) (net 12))
 (segment (start 147.042 106.8707) (end 151.3433 111.172) (width 0.5588) (layer F.Cu) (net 13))
 (segment (start 140.97 106.8707) (end 147.042 106.8707) (width 0.5588) (layer F.Cu) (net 13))
 (segment (start 140.97 105.41) (end 140.97 106.8707) (width 0.5588) (layer F.Cu) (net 13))
 (segment (start 152.654 111.172) (end 151.3433 111.172) (width 0.5588) (layer F.Cu) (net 13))
 (segment (start 173.4793 118.146) (end 173.5153 118.11) (width 0.5588) (layer F.Cu) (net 15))
 (segment (start 170.853 118.146) (end 173.4793 118.146) (width 0.5588) (layer F.Cu) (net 15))
 (segment (start 174.926 118.11) (end 173.5153 118.11) (width 0.5588) (layer F.Cu) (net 15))
 (segment (start 162.903 118.146) (end 162.903 117.4906) (width 0.5588) (layer F.Cu) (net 15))
 (segment (start 168.7619 117.4906) (end 169.4173 118.146) (width 0.5588) (layer F.Cu) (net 15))
 (segment (start 162.903 117.4906) (end 168.7619 117.4906) (width 0.5588) (layer F.Cu) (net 15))
 (segment (start 170.853 118.146) (end 169.4173 118.146) (width 0.5588) (layer F.Cu) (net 15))
 (segment (start 162.4813 117.4906) (end 162.903 117.4906) (width 0.5588) (layer F.Cu) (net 15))
 (segment (start 150.4007 105.41) (end 162.4813 117.4906) (width 0.5588) (layer F.Cu) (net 15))
 (segment (start 148.59 105.41) (end 150.4007 105.41) (width 0.5588) (layer F.Cu) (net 15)))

